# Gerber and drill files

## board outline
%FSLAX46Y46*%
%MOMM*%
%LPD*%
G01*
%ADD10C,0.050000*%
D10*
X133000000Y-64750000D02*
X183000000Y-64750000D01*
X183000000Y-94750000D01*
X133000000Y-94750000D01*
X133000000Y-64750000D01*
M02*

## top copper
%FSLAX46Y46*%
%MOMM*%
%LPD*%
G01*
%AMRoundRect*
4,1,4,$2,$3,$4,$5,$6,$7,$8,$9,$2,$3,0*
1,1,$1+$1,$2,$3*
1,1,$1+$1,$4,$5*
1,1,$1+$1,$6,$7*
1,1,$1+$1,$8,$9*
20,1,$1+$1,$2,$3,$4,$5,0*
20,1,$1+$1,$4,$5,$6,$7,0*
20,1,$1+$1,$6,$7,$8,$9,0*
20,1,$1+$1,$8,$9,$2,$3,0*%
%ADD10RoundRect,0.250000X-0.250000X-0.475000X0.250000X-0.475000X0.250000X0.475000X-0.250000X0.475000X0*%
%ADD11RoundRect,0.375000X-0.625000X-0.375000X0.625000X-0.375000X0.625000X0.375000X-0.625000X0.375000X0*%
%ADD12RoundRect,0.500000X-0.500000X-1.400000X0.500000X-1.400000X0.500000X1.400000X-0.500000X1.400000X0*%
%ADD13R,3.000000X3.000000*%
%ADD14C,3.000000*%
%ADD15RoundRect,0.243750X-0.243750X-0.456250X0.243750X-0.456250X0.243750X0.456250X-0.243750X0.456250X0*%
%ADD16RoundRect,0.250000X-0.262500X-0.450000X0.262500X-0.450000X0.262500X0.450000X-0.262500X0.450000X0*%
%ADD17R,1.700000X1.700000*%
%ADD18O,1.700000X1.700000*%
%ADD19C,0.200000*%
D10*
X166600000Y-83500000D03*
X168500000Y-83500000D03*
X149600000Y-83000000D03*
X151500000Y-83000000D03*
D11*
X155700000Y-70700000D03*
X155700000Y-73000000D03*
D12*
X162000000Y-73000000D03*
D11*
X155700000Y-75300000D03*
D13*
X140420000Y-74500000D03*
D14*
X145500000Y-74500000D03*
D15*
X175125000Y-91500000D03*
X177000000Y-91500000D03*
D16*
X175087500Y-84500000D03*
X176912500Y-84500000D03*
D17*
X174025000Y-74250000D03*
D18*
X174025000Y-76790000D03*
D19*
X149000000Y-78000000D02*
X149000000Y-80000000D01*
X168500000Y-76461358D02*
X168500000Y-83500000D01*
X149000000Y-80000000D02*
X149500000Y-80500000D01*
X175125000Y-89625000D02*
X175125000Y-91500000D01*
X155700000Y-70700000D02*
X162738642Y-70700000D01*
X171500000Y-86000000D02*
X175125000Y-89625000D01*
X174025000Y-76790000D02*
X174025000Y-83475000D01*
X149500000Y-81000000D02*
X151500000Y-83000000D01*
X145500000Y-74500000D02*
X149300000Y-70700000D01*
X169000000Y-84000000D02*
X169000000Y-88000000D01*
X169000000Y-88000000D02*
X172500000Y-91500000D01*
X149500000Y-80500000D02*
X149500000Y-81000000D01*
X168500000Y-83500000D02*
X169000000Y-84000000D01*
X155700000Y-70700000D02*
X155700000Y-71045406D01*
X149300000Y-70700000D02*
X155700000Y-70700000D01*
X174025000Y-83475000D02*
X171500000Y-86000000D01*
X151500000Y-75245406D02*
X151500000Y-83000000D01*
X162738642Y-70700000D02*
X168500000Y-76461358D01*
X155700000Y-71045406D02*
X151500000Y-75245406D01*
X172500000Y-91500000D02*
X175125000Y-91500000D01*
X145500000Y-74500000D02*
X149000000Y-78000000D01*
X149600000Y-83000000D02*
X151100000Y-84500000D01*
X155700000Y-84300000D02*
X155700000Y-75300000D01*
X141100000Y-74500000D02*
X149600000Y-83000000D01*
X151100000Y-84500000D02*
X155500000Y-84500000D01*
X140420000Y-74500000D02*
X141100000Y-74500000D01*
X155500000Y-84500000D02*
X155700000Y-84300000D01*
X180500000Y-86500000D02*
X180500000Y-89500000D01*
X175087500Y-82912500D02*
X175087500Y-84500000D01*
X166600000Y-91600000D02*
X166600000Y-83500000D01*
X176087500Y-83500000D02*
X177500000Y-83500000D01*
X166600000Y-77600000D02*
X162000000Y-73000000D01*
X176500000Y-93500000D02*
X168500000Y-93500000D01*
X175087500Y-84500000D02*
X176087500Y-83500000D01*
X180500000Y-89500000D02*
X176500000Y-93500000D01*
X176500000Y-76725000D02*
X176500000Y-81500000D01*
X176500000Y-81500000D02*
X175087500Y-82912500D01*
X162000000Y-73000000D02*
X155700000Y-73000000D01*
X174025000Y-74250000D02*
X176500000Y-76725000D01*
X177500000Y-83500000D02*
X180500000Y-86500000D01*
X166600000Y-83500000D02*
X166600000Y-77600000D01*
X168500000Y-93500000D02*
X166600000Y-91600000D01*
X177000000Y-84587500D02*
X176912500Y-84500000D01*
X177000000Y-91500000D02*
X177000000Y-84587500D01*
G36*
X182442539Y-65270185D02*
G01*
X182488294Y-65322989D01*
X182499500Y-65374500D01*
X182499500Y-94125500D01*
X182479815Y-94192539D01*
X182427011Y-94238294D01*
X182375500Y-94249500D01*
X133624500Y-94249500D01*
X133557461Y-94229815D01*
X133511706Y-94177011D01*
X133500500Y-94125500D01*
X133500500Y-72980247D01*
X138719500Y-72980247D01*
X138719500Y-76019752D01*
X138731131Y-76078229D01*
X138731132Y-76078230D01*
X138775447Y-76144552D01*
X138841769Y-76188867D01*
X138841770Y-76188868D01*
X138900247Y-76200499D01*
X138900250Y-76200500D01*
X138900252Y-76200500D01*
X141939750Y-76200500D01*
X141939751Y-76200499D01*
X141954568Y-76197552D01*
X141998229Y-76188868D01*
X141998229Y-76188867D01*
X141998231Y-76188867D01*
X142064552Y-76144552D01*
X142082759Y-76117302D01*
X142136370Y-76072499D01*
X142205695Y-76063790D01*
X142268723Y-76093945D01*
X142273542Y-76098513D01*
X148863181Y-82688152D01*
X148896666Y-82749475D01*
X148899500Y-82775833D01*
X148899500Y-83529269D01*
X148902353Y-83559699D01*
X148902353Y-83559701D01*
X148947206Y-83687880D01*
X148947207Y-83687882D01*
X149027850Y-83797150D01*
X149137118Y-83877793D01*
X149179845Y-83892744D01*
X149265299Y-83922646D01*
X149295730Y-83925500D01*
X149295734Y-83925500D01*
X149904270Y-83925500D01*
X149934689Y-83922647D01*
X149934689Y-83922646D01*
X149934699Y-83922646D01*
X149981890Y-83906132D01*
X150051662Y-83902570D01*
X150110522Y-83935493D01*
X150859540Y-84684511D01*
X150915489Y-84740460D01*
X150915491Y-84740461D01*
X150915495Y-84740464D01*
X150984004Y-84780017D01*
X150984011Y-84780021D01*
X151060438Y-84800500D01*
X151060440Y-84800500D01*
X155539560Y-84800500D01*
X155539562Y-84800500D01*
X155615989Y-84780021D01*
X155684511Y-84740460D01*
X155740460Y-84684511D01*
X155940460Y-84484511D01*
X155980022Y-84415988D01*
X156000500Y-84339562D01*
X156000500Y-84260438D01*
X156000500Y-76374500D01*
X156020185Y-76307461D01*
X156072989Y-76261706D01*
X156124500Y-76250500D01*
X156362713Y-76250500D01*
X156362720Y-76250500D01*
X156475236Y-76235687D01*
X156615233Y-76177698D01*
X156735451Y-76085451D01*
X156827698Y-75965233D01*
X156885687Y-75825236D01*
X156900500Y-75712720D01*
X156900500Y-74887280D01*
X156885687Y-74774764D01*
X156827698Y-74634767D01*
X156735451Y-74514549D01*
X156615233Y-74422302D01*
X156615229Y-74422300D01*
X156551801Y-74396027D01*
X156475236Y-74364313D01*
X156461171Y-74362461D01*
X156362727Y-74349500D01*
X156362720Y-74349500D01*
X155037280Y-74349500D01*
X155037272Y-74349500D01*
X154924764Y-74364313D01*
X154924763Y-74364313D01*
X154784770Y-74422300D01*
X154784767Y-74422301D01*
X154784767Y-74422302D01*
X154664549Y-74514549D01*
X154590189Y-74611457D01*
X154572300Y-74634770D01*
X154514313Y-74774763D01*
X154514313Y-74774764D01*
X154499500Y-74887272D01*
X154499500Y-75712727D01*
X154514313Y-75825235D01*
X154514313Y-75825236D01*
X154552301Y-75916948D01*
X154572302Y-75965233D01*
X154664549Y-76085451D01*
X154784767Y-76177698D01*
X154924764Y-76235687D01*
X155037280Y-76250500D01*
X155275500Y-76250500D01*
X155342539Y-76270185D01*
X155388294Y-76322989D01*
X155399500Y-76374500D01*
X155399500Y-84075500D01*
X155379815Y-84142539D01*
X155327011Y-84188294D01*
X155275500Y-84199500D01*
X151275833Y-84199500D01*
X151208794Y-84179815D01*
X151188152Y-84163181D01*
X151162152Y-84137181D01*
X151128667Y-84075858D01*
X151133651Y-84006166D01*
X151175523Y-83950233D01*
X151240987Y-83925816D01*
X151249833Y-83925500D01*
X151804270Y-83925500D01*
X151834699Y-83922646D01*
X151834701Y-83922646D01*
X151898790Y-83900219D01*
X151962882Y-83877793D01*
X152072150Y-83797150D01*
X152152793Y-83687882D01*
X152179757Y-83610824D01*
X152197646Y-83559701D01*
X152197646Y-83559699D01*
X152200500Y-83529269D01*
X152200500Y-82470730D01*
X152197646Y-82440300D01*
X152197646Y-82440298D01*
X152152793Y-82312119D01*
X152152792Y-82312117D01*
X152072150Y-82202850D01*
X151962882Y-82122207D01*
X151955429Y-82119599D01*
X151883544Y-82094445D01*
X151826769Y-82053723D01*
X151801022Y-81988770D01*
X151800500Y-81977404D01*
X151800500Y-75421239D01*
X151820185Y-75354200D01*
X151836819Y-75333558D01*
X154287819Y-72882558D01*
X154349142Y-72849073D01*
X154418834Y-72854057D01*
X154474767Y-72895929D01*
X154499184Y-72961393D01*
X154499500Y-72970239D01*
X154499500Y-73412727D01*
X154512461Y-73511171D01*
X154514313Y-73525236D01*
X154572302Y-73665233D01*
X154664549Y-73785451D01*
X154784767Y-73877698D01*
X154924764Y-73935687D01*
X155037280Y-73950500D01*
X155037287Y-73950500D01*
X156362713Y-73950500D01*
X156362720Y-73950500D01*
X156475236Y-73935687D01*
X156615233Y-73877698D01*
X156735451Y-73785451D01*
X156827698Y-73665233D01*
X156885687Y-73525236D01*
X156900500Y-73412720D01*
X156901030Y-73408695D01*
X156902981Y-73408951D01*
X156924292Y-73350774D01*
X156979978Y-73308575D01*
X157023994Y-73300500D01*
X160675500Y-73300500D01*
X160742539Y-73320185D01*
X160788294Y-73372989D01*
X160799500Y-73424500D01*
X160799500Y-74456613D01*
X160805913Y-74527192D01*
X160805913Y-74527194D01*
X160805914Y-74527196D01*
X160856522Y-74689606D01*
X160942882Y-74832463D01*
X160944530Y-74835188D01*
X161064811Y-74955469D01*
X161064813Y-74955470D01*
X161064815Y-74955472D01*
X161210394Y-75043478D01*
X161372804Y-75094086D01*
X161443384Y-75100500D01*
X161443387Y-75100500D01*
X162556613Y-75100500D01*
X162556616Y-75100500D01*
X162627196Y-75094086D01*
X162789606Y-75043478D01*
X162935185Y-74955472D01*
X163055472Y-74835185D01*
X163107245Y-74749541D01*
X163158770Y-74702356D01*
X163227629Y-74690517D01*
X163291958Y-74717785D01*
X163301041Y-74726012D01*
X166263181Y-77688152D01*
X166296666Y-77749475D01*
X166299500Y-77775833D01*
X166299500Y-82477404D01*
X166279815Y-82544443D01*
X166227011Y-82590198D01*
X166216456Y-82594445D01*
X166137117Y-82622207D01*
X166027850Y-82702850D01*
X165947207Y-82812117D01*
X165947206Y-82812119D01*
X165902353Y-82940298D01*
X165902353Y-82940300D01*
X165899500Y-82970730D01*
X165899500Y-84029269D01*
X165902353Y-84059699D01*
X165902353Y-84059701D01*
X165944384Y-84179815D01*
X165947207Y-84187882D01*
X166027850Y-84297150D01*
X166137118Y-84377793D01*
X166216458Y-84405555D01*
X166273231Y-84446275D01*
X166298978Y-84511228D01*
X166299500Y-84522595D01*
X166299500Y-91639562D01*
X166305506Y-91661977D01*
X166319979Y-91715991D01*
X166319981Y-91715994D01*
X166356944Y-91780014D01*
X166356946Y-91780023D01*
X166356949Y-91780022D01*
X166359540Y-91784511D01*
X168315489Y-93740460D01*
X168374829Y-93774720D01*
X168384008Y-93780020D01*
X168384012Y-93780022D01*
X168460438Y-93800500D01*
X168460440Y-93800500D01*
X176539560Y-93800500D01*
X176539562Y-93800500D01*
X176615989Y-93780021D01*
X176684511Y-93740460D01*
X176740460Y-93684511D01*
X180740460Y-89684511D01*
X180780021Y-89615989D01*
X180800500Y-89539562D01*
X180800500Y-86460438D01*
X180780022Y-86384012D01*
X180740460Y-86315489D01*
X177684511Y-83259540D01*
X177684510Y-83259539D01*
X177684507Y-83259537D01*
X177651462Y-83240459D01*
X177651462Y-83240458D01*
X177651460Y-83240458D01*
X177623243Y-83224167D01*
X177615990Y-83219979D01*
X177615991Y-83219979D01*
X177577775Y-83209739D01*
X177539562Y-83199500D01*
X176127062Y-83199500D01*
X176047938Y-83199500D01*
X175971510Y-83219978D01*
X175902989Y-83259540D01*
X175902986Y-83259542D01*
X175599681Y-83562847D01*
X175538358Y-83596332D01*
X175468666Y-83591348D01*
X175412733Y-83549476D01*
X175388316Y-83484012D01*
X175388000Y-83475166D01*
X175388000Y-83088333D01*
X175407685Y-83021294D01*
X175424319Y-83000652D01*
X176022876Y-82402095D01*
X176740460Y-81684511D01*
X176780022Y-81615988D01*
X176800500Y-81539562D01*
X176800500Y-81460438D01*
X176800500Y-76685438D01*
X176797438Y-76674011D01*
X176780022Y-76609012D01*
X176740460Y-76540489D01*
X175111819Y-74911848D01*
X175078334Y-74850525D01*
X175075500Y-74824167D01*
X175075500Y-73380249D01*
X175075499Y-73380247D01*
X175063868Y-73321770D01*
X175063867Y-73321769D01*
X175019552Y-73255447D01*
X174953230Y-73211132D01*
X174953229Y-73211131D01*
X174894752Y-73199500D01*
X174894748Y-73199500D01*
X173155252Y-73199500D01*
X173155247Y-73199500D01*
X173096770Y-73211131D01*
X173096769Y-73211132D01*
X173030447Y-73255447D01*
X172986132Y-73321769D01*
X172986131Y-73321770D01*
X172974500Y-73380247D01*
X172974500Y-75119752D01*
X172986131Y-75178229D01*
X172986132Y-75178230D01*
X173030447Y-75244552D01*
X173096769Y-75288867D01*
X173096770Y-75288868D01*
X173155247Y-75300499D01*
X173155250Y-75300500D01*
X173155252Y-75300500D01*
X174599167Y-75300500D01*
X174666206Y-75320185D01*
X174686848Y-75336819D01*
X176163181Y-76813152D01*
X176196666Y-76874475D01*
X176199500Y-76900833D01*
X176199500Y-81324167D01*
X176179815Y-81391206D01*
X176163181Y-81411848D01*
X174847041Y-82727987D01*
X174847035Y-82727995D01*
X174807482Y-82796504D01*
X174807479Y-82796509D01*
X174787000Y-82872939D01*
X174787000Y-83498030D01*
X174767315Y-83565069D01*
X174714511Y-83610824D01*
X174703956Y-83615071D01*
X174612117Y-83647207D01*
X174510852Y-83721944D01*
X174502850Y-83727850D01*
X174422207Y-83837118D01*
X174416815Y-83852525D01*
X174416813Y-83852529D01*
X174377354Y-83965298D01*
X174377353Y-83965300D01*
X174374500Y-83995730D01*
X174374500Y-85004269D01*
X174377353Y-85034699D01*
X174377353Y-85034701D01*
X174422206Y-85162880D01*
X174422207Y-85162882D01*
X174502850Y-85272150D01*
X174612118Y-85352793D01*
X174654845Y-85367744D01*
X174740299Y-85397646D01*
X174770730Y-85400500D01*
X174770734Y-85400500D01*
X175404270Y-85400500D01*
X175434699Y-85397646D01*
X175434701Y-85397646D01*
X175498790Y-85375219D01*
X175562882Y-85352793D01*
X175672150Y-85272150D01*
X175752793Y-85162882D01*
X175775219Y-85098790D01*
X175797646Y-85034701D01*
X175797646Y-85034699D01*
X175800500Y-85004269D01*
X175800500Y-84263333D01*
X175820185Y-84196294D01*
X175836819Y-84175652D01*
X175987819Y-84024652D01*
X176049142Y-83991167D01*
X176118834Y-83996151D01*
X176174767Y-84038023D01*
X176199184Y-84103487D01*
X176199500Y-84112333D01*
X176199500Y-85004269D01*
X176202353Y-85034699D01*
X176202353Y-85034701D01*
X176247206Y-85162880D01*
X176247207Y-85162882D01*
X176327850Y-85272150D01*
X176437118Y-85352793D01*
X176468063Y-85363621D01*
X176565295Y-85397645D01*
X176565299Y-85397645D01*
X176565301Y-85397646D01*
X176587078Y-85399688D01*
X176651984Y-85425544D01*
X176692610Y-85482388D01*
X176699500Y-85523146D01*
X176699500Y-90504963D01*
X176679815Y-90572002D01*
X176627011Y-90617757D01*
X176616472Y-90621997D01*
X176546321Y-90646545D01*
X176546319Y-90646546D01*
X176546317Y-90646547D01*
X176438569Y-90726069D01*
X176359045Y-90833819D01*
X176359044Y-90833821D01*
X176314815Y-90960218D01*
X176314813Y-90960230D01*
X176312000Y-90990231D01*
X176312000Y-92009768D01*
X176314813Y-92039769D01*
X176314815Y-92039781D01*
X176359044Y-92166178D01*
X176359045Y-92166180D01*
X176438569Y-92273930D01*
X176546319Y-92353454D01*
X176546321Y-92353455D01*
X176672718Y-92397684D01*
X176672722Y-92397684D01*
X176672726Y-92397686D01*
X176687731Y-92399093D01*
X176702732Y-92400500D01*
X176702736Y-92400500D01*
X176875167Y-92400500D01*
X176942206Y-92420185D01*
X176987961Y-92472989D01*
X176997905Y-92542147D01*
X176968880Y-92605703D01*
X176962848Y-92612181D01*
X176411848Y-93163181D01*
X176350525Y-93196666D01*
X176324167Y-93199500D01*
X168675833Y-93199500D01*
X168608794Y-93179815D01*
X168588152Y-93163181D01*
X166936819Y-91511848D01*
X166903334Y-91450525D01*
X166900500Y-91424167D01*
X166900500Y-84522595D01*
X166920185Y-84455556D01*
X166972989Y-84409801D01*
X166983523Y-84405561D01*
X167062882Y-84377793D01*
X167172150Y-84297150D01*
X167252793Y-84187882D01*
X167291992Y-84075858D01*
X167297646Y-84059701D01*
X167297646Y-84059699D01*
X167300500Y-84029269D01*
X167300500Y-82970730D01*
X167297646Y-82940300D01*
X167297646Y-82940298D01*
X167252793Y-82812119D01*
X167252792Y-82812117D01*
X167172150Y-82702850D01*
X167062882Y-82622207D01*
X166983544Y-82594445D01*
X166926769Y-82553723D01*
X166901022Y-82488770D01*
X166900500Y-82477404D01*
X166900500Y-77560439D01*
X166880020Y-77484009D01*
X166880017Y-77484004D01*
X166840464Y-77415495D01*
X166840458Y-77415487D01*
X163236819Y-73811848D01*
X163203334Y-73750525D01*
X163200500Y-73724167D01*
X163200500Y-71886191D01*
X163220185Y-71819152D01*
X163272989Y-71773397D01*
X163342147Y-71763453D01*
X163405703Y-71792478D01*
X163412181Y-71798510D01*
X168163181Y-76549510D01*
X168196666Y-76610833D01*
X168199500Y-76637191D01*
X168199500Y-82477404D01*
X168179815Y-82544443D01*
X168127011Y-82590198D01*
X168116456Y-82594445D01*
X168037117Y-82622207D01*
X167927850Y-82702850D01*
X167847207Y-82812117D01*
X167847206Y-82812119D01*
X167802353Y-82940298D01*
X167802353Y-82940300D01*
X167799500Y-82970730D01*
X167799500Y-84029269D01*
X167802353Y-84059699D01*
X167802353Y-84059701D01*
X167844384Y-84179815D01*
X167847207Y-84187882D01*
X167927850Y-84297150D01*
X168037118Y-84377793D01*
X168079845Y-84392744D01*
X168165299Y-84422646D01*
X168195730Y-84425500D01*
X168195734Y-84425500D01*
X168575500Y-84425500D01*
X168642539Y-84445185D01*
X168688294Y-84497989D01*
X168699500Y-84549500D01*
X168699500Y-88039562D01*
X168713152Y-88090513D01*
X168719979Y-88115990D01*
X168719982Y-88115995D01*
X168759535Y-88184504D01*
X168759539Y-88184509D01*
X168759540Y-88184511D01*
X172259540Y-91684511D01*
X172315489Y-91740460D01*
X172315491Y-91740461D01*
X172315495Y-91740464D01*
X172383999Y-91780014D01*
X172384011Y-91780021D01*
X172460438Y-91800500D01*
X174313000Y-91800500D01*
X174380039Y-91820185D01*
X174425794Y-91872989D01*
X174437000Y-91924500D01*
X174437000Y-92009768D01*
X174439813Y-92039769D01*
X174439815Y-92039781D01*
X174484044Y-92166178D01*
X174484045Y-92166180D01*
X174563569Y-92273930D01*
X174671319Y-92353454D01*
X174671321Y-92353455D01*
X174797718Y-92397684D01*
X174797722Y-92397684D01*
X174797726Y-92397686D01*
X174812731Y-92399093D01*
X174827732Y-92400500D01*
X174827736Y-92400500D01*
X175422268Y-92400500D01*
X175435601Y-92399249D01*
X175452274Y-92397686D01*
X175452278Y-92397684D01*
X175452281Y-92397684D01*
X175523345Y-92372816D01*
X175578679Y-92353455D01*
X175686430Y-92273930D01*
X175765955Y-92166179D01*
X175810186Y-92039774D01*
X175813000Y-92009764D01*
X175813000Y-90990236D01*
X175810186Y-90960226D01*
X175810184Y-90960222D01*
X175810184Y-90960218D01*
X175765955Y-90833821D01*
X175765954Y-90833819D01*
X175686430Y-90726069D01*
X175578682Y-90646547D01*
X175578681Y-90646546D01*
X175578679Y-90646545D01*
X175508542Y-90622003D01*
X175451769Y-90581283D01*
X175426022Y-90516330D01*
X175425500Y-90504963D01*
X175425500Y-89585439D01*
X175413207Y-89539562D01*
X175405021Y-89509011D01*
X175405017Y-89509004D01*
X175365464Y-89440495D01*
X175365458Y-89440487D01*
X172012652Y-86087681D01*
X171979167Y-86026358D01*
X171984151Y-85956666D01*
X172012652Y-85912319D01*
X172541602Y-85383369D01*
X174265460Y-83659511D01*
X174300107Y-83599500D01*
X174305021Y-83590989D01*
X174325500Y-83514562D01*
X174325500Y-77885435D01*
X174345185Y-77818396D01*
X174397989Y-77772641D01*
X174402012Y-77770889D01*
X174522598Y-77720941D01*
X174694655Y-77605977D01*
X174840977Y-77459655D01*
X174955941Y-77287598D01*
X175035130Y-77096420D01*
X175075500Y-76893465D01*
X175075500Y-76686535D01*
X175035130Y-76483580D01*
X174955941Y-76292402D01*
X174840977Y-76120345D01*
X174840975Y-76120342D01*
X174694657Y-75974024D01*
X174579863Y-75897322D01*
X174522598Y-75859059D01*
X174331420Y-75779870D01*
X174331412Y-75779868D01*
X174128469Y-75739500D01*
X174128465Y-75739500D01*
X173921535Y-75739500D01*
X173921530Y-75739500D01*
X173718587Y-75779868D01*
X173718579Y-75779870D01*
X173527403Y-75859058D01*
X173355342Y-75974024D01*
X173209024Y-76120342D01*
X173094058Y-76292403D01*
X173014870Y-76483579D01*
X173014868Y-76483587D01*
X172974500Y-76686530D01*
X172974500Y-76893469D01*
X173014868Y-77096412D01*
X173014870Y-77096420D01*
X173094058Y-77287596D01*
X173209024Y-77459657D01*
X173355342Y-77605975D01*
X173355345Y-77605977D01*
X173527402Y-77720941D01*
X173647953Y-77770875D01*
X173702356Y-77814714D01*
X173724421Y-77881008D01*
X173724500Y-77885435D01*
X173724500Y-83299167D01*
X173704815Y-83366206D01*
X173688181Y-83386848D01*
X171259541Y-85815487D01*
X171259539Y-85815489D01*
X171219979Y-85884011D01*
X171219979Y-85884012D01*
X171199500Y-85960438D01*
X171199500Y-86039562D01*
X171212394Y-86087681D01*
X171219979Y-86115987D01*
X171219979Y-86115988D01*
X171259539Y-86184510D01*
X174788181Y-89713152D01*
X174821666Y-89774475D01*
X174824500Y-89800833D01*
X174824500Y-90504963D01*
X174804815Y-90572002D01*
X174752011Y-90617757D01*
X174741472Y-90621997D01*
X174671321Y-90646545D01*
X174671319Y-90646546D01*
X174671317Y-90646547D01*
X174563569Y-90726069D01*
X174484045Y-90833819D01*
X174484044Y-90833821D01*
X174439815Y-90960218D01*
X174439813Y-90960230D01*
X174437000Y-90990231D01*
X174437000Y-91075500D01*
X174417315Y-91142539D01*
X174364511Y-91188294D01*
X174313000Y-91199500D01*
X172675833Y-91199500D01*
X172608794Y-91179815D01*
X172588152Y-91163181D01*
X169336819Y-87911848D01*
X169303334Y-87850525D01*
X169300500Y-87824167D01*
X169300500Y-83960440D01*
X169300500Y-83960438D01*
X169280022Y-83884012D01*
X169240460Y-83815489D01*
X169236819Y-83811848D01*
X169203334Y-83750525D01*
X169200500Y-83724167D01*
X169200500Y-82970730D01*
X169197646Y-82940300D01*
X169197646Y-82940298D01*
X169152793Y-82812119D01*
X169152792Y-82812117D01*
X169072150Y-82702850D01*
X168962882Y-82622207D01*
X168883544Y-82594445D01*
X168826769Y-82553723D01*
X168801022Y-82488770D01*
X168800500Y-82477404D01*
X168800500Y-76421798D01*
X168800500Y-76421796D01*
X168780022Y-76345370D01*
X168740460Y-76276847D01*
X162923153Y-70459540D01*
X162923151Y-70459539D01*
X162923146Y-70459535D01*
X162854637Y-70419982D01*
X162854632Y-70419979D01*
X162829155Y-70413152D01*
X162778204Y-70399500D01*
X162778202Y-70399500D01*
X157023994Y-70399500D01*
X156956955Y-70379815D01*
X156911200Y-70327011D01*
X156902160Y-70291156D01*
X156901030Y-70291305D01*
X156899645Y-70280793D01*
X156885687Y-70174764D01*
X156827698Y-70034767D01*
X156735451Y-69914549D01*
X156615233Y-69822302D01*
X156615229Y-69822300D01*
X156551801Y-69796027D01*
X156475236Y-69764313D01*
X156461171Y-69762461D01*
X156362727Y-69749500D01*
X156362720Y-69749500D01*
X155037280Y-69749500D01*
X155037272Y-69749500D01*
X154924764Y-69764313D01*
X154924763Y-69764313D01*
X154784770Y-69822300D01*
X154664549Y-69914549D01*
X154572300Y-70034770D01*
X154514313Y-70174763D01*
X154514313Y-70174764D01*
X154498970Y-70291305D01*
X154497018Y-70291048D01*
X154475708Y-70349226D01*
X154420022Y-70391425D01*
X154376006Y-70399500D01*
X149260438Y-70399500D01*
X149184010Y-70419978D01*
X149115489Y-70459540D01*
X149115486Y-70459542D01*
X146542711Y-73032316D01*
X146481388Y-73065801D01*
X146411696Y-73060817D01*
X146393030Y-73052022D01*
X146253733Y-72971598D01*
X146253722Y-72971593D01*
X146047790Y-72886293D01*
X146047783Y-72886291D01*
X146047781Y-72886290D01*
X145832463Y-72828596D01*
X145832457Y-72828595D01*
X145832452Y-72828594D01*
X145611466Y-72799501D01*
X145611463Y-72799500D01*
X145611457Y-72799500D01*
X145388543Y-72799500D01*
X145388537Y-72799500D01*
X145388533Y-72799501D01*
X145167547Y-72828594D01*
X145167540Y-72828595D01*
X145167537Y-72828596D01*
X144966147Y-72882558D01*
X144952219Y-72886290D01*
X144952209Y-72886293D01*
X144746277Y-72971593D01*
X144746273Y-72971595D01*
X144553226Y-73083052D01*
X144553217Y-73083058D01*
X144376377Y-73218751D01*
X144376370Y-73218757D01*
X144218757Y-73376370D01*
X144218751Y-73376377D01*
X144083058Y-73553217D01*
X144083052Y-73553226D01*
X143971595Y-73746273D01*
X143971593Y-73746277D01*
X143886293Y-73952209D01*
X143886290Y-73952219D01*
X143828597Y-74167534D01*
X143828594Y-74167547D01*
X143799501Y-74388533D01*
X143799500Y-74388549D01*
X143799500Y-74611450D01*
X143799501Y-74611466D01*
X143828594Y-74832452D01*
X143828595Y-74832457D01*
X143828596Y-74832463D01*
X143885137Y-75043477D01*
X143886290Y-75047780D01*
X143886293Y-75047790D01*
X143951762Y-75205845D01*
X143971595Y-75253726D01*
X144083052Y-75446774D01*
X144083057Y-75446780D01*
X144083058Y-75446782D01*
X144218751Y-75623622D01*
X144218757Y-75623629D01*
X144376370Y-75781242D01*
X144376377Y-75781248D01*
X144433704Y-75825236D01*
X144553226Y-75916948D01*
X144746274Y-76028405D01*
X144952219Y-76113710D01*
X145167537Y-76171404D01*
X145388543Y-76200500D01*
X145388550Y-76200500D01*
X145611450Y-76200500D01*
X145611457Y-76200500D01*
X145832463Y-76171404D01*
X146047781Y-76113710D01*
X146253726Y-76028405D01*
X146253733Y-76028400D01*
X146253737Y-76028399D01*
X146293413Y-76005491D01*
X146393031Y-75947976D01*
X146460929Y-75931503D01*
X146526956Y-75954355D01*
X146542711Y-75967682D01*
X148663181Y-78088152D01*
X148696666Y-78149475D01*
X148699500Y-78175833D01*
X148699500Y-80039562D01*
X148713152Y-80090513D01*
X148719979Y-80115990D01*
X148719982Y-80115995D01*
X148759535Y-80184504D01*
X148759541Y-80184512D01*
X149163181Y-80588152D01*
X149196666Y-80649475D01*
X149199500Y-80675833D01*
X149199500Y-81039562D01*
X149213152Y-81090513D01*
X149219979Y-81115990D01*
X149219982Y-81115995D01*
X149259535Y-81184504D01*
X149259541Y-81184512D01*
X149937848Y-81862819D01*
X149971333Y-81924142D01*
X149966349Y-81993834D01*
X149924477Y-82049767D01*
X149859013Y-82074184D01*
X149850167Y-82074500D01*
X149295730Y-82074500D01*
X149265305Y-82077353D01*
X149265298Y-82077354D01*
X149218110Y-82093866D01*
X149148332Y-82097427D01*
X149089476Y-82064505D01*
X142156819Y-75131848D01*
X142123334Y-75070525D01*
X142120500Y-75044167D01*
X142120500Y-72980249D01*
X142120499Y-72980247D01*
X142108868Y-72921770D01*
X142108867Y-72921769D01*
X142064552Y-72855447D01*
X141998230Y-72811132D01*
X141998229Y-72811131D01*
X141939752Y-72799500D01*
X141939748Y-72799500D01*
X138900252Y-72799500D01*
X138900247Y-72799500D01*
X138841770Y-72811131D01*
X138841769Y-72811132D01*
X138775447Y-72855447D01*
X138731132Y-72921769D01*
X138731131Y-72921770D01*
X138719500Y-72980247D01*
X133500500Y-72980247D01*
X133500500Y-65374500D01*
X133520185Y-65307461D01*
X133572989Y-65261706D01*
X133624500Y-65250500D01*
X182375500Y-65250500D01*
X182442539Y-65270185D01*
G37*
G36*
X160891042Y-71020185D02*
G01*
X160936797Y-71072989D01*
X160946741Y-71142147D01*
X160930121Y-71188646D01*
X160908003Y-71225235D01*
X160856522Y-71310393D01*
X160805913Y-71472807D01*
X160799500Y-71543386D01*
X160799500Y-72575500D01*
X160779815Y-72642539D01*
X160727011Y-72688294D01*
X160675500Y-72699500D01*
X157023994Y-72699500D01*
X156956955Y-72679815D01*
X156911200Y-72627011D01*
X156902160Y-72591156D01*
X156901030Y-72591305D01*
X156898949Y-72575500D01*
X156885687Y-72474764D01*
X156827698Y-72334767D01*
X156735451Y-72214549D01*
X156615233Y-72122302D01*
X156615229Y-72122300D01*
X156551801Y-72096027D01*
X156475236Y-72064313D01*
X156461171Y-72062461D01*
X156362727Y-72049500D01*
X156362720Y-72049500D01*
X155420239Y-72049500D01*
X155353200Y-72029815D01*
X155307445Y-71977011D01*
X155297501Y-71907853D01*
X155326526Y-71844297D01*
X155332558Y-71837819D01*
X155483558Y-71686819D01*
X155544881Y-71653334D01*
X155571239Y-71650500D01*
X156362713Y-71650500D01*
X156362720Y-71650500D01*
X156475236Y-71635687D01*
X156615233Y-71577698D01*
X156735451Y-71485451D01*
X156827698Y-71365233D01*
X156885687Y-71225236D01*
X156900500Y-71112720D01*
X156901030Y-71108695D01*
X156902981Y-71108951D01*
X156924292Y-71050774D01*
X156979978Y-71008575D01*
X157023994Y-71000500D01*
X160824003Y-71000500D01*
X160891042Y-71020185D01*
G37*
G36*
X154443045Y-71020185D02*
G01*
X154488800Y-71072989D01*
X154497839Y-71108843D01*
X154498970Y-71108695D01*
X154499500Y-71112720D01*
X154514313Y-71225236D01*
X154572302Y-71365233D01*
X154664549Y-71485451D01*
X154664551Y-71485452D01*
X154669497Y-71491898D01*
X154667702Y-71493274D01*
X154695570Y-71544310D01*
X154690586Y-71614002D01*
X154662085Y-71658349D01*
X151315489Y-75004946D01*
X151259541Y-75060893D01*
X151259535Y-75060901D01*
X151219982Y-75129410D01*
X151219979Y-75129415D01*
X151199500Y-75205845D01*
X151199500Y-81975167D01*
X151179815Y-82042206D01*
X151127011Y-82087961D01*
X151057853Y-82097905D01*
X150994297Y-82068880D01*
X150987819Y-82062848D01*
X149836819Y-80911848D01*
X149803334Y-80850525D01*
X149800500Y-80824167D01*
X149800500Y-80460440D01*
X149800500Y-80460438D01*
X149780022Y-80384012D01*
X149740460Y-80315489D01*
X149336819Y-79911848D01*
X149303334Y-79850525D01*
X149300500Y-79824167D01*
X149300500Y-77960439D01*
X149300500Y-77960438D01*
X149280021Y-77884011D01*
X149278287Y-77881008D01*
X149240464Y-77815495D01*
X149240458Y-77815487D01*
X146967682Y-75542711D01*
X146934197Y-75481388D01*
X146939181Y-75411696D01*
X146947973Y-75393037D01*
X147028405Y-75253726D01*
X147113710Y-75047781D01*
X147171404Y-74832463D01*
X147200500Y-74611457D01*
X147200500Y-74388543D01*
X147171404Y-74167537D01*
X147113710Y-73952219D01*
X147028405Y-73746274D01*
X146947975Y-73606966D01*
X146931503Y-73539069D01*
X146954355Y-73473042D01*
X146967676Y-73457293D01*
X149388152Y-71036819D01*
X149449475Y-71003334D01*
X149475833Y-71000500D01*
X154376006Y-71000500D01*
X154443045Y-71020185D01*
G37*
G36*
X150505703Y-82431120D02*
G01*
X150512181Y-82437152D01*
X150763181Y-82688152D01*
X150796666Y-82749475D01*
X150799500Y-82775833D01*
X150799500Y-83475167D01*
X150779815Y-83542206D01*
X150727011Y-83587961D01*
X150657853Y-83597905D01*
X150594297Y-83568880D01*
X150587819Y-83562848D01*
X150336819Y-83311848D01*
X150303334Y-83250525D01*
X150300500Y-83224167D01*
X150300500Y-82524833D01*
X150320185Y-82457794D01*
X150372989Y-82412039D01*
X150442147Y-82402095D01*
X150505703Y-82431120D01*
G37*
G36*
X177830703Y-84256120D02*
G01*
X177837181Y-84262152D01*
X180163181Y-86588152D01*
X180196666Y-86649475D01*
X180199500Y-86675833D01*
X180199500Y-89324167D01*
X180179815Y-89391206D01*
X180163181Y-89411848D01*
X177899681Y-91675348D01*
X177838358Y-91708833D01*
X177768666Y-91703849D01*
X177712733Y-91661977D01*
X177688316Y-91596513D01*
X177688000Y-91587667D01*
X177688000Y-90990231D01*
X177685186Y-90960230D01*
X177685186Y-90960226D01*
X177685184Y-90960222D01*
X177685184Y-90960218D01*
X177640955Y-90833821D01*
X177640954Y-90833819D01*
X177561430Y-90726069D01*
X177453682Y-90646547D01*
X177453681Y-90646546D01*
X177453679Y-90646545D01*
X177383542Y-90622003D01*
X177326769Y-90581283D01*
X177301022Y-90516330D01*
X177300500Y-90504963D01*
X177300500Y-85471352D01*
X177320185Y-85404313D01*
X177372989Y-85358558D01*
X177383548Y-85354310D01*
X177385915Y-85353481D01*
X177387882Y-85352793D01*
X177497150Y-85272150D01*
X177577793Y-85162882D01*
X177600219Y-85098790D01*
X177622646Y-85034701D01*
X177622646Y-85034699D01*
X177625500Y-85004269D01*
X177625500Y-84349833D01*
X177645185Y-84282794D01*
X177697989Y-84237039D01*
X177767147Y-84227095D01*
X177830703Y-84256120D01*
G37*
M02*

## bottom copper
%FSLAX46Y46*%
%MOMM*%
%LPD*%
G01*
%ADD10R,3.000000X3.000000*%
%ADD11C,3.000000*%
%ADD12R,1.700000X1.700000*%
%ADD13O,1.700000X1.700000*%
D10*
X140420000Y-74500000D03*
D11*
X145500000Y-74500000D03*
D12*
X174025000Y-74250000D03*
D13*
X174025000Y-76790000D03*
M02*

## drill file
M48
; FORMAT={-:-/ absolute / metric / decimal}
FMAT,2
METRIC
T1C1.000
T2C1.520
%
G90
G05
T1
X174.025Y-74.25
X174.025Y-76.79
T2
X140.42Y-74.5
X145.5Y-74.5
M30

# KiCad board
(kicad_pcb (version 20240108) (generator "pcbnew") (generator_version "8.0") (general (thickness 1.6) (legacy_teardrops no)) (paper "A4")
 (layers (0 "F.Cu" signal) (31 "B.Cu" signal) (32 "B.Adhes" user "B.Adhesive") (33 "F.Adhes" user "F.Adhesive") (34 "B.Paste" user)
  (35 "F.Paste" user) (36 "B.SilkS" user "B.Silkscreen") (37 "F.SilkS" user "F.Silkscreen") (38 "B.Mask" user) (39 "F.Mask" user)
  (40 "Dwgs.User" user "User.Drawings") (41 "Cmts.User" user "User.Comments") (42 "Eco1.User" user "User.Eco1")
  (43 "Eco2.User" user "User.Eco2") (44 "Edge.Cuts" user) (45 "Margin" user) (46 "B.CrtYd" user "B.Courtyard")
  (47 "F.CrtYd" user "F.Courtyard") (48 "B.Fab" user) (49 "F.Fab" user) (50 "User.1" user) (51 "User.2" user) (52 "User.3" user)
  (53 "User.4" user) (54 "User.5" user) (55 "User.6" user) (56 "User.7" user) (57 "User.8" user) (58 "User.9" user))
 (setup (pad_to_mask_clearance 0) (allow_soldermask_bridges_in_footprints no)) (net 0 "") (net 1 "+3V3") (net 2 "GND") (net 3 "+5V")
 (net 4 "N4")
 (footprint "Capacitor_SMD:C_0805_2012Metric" (layer "F.Cu") (at 167.55 83.5)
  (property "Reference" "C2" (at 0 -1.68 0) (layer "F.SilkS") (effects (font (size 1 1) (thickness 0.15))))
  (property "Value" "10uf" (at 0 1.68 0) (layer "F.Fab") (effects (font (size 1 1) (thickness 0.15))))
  (pad "1" smd roundrect (at -0.95 0) (size 1 1.45) (layers "F.Cu" "F.Paste" "F.Mask") (roundrect_rratio 0.25) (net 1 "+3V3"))
  (pad "2" smd roundrect (at 0.95 0) (size 1 1.45) (layers "F.Cu" "F.Paste" "F.Mask") (roundrect_rratio 0.25) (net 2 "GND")))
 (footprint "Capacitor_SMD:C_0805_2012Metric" (layer "F.Cu") (at 150.55 83)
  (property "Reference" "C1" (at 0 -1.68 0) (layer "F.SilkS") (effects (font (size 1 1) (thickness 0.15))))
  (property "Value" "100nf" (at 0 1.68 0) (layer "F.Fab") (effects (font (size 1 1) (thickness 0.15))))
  (pad "1" smd roundrect (at -0.95 0) (size 1 1.45) (layers "F.Cu" "F.Paste" "F.Mask") (roundrect_rratio 0.25) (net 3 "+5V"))
  (pad "2" smd roundrect (at 0.95 0) (size 1 1.45) (layers "F.Cu" "F.Paste" "F.Mask") (roundrect_rratio 0.25) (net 2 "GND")))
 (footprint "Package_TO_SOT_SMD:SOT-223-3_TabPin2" (layer "F.Cu") (at 158.85 73)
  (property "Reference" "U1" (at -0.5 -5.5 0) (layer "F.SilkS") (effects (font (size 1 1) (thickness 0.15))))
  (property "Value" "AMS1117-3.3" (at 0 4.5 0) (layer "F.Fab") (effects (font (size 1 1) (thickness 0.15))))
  (pad "1" smd roundrect (at -3.15 -2.3) (size 2 1.5) (layers "F.Cu" "F.Paste" "F.Mask") (roundrect_rratio 0.25) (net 2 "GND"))
  (pad "2" smd roundrect (at -3.15 0) (size 2 1.5) (layers "F.Cu" "F.Paste" "F.Mask") (roundrect_rratio 0.25) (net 1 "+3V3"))
  (pad "2" smd roundrect (at 3.15 0) (size 2 3.8) (layers "F.Cu" "F.Paste" "F.Mask") (roundrect_rratio 0.25) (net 1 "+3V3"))
  (pad "3" smd roundrect (at -3.15 2.3) (size 2 1.5) (layers "F.Cu" "F.Paste" "F.Mask") (roundrect_rratio 0.25) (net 3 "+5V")))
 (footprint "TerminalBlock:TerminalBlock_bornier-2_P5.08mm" (layer "F.Cu") (at 140.42 74.5)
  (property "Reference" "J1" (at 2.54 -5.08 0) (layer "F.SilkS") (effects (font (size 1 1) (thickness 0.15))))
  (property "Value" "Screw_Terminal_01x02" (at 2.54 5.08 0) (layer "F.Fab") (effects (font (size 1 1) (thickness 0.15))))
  (pad "1" thru_hole rect (at 0 0) (size 3 3) (drill 1.52) (layers "*.Cu" "*.Mask") (remove_unused_layers no) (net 3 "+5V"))
  (pad "2" thru_hole circle (at 5.08 0) (size 3 3) (drill 1.52) (layers "*.Cu" "*.Mask") (remove_unused_layers no) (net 2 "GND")))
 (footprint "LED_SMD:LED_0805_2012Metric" (layer "F.Cu") (at 176.0625 91.5)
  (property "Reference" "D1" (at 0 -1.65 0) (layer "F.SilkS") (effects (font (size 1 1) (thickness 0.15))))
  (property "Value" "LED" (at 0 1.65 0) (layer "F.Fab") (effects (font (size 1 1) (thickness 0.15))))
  (pad "1" smd roundrect (at -0.9375 0) (size 0.975 1.4) (layers "F.Cu" "F.Paste" "F.Mask") (roundrect_rratio 0.25) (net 2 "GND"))
  (pad "2" smd roundrect (at 0.9375 0) (size 0.975 1.4) (layers "F.Cu" "F.Paste" "F.Mask") (roundrect_rratio 0.25) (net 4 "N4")))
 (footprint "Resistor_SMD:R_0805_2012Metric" (layer "F.Cu") (at 176 84.5)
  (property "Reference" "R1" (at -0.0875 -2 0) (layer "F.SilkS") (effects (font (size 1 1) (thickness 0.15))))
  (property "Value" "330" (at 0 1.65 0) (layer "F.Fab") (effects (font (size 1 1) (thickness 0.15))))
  (pad "1" smd roundrect (at -0.9125 0) (size 1.025 1.4) (layers "F.Cu" "F.Paste" "F.Mask") (roundrect_rratio 0.243902) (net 1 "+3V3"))
  (pad "2" smd roundrect (at 0.9125 0) (size 1.025 1.4) (layers "F.Cu" "F.Paste" "F.Mask") (roundrect_rratio 0.243902) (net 4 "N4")))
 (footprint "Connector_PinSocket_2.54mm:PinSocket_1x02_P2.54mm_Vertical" (layer "F.Cu") (at 174.025 74.25)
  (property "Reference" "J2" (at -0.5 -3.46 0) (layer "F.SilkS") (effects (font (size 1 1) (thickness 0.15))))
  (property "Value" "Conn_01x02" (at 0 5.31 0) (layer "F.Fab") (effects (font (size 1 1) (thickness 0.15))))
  (pad "1" thru_hole rect (at 0 0) (size 1.7 1.7) (drill 1) (layers "*.Cu" "*.Mask") (remove_unused_layers no) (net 1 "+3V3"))
  (pad "2" thru_hole oval (at 0 2.54) (size 1.7 1.7) (drill 1) (layers "*.Cu" "*.Mask") (remove_unused_layers no) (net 2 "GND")))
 (gr_rect (start 133 64.75) (end 183 94.75) (locked yes) (stroke (width 0.05) (type default)) (fill none) (layer "Edge.Cuts"))
 (segment (start 149 78) (end 149 80) (width 0.2) (layer "F.Cu") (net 2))
 (segment (start 168.5 76.461358) (end 168.5 83.5) (width 0.2) (layer "F.Cu") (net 2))
 (segment (start 149 80) (end 149.5 80.5) (width 0.2) (layer "F.Cu") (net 2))
 (segment (start 175.125 89.625) (end 175.125 91.5) (width 0.2) (layer "F.Cu") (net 2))
 (segment (start 155.7 70.7) (end 162.738642 70.7) (width 0.2) (layer "F.Cu") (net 2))
 (segment (start 171.5 86) (end 175.125 89.625) (width 0.2) (layer "F.Cu") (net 2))
 (segment (start 174.025 76.79) (end 174.025 83.475) (width 0.2) (layer "F.Cu") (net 2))
 (segment (start 149.5 81) (end 151.5 83) (width 0.2) (layer "F.Cu") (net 2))
 (segment (start 145.5 74.5) (end 149.3 70.7) (width 0.2) (layer "F.Cu") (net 2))
 (segment (start 169 84) (end 169 88) (width 0.2) (layer "F.Cu") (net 2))
 (segment (start 169 88) (end 172.5 91.5) (width 0.2) (layer "F.Cu") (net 2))
 (segment (start 149.5 80.5) (end 149.5 81) (width 0.2) (layer "F.Cu") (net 2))
 (segment (start 168.5 83.5) (end 169 84) (width 0.2) (layer "F.Cu") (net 2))
 (segment (start 155.7 70.7) (end 155.7 71.045406) (width 0.2) (layer "F.Cu") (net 2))
 (segment (start 149.3 70.7) (end 155.7 70.7) (width 0.2) (layer "F.Cu") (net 2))
 (segment (start 174.025 83.475) (end 171.5 86) (width 0.2) (layer "F.Cu") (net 2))
 (segment (start 151.5 75.245406) (end 151.5 83) (width 0.2) (layer "F.Cu") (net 2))
 (segment (start 162.738642 70.7) (end 168.5 76.461358) (width 0.2) (layer "F.Cu") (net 2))
 (segment (start 155.7 71.045406) (end 151.5 75.245406) (width 0.2) (layer "F.Cu") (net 2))
 (segment (start 172.5 91.5) (end 175.125 91.5) (width 0.2) (layer "F.Cu") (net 2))
 (segment (start 145.5 74.5) (end 149 78) (width 0.2) (layer "F.Cu") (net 2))
 (segment (start 149.6 83) (end 151.1 84.5) (width 0.2) (layer "F.Cu") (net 3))
 (segment (start 155.7 84.3) (end 155.7 75.3) (width 0.2) (layer "F.Cu") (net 3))
 (segment (start 141.1 74.5) (end 149.6 83) (width 0.2) (layer "F.Cu") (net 3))
 (segment (start 151.1 84.5) (end 155.5 84.5) (width 0.2) (layer "F.Cu") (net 3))
 (segment (start 140.42 74.5) (end 141.1 74.5) (width 0.2) (layer "F.Cu") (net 3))
 (segment (start 155.5 84.5) (end 155.7 84.3) (width 0.2) (layer "F.Cu") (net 3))
 (segment (start 180.5 86.5) (end 180.5 89.5) (width 0.2) (layer "F.Cu") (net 1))
 (segment (start 175.0875 82.9125) (end 175.0875 84.5) (width 0.2) (layer "F.Cu") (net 1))
 (segment (start 166.6 91.6) (end 166.6 83.5) (width 0.2) (layer "F.Cu") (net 1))
 (segment (start 176.0875 83.5) (end 177.5 83.5) (width 0.2) (layer "F.Cu") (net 1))
 (segment (start 166.6 77.6) (end 162 73) (width 0.2) (layer "F.Cu") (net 1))
 (segment (start 176.5 93.5) (end 168.5 93.5) (width 0.2) (layer "F.Cu") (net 1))
 (segment (start 175.0875 84.5) (end 176.0875 83.5) (width 0.2) (layer "F.Cu") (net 1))
 (segment (start 180.5 89.5) (end 176.5 93.5) (width 0.2) (layer "F.Cu") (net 1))
 (segment (start 176.5 76.725) (end 176.5 81.5) (width 0.2) (layer "F.Cu") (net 1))
 (segment (start 176.5 81.5) (end 175.0875 82.9125) (width 0.2) (layer "F.Cu") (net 1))
 (segment (start 162 73) (end 155.7 73) (width 0.2) (layer "F.Cu") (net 1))
 (segment (start 174.025 74.25) (end 176.5 76.725) (width 0.2) (layer "F.Cu") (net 1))
 (segment (start 177.5 83.5) (end 180.5 86.5) (width 0.2) (layer "F.Cu") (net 1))
 (segment (start 166.6 83.5) (end 166.6 77.6) (width 0.2) (layer "F.Cu") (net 1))
 (segment (start 168.5 93.5) (end 166.6 91.6) (width 0.2) (layer "F.Cu") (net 1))
 (segment (start 177 84.5875) (end 176.9125 84.5) (width 0.2) (layer "F.Cu") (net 4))
 (segment (start 177 91.5) (end 177 84.5875) (width 0.2) (layer "F.Cu") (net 4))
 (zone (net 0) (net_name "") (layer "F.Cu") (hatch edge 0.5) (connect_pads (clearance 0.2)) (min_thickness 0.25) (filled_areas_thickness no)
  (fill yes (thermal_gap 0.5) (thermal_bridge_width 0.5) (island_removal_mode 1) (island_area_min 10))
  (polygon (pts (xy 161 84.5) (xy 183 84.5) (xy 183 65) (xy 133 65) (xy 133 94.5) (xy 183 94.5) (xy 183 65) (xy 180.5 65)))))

